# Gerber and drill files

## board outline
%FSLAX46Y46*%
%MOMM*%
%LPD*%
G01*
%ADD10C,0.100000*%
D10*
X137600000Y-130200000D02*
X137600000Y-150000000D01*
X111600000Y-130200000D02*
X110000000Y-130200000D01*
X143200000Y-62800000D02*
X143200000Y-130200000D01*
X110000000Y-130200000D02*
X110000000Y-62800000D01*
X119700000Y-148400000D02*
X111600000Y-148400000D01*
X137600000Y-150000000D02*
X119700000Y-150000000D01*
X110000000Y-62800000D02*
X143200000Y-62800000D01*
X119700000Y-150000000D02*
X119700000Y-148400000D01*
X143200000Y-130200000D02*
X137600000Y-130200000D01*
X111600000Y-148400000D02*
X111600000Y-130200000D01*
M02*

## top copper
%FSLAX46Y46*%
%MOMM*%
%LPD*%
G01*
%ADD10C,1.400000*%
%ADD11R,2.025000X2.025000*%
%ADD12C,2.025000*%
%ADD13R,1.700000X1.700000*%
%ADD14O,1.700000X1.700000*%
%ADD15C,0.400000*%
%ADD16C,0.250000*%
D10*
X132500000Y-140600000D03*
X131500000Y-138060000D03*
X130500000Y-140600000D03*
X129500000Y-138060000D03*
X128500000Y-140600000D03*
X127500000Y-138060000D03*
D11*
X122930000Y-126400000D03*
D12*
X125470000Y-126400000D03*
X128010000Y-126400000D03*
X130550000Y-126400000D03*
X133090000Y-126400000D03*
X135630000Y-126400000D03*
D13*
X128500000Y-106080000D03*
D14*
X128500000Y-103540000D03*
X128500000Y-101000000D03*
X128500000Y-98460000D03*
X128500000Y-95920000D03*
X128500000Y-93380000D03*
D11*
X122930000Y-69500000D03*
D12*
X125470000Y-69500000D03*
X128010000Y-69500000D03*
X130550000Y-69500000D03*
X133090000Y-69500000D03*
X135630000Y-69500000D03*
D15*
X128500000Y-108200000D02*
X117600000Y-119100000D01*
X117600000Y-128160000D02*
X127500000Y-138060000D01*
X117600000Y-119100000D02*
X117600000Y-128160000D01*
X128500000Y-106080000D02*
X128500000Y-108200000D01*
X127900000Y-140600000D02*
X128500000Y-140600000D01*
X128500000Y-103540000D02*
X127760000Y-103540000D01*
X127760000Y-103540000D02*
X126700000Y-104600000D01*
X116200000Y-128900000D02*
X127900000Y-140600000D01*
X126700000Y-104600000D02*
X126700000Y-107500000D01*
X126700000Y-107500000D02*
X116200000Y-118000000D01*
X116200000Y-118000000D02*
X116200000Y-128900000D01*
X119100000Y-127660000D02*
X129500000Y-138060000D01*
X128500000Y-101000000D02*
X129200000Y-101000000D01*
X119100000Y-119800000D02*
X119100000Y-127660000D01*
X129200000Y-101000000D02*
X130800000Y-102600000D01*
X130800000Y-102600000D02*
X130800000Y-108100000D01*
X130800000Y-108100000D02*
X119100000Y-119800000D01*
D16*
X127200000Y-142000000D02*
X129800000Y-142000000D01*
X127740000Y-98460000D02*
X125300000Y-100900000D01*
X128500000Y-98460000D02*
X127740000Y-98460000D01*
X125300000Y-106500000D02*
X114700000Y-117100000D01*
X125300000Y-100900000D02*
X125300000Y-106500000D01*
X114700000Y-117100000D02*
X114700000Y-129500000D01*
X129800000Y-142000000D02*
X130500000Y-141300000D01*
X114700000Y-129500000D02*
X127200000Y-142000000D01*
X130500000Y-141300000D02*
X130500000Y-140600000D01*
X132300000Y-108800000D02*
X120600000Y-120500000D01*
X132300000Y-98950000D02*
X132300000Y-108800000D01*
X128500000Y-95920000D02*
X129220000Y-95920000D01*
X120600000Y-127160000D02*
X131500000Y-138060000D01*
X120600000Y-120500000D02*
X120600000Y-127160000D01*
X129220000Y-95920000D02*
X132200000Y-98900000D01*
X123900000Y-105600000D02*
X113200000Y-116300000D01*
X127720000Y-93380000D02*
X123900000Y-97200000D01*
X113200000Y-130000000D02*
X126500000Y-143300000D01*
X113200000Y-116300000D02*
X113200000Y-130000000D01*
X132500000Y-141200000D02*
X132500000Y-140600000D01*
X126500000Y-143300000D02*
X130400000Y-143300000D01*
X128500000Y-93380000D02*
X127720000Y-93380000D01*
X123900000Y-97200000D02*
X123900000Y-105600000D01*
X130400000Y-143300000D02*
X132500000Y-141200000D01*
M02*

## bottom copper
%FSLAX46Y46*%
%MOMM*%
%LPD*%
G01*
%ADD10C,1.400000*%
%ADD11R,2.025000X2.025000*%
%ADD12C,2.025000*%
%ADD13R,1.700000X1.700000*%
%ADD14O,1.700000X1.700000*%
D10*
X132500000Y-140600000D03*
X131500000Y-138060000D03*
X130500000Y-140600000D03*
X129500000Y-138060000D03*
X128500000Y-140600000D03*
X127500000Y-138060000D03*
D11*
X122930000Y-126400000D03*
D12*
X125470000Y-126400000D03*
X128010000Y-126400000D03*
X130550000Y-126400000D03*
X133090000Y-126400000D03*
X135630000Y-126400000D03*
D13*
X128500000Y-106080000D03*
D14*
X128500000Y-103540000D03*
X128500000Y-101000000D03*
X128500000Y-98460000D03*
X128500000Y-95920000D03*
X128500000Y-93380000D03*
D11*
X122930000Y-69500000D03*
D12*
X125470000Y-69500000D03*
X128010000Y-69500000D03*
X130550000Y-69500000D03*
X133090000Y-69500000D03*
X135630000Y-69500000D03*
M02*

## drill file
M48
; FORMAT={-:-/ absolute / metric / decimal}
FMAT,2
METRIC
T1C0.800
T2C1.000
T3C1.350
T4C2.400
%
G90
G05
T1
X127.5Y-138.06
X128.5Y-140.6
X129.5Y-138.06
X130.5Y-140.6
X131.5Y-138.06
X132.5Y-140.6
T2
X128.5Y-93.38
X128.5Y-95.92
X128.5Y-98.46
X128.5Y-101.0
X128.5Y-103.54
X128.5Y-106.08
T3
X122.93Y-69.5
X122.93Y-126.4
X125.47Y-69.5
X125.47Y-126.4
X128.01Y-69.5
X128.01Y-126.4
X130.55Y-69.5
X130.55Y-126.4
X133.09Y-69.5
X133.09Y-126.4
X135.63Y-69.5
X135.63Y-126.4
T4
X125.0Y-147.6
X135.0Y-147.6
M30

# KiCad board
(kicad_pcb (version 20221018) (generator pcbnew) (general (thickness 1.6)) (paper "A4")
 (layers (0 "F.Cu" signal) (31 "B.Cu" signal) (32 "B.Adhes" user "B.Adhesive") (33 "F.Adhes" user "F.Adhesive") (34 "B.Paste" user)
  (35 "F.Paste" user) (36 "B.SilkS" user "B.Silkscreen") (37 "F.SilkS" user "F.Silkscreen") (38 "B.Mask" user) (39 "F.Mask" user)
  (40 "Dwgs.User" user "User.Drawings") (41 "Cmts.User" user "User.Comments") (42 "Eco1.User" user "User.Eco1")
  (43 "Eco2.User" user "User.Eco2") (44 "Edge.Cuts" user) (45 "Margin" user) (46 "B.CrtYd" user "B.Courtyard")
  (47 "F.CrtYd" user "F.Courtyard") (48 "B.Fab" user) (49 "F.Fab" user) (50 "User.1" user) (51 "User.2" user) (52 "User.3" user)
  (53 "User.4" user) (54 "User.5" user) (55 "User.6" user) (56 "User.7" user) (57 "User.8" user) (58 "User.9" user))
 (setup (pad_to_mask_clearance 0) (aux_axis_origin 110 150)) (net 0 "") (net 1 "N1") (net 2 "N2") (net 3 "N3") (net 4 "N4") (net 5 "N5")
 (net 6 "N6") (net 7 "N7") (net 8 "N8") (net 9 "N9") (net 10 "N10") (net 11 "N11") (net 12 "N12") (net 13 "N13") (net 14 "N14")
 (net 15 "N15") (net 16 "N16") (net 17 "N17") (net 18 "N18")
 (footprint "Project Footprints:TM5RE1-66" (layer "B.Cu") (at 130 147.6 180)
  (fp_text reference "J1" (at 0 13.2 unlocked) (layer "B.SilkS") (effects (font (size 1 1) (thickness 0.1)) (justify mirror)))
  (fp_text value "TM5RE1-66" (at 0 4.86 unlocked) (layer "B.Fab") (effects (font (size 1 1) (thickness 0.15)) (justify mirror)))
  (pad "" np_thru_hole circle (at -5 0 180) (size 2.4 2.4) (drill 2.4) (layers "F&B.Cu" "*.Mask"))
  (pad "" np_thru_hole circle (at 5 0 180) (size 2.4 2.4) (drill 2.4) (layers "F&B.Cu" "*.Mask"))
  (pad "1" thru_hole circle (at -2.5 7 180) (size 1.4 1.4) (drill 0.8) (layers "*.Cu" "*.Mask") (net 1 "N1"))
  (pad "2" thru_hole circle (at -1.5 9.54 180) (size 1.4 1.4) (drill 0.8) (layers "*.Cu" "*.Mask") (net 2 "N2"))
  (pad "3" thru_hole circle (at -0.5 7 180) (size 1.4 1.4) (drill 0.8) (layers "*.Cu" "*.Mask") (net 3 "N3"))
  (pad "4" thru_hole circle (at 0.5 9.54 180) (size 1.4 1.4) (drill 0.8) (layers "*.Cu" "*.Mask") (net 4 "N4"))
  (pad "5" thru_hole circle (at 1.5 7 180) (size 1.4 1.4) (drill 0.8) (layers "*.Cu" "*.Mask") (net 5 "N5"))
  (pad "6" thru_hole circle (at 2.5 9.54 180) (size 1.4 1.4) (drill 0.8) (layers "*.Cu" "*.Mask") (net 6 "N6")))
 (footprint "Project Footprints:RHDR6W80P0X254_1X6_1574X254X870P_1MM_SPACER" (layer "B.Cu") (at 122.93 126.4)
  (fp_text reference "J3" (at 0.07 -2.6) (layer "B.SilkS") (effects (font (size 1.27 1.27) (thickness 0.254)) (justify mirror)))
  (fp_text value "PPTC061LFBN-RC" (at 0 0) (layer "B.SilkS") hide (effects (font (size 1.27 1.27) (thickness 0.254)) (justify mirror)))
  (pad "1" thru_hole rect (at 0 0) (size 2.025 2.025) (drill 1.35) (layers "*.Cu" "*.Mask") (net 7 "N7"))
  (pad "2" thru_hole circle (at 2.54 0) (size 2.025 2.025) (drill 1.35) (layers "*.Cu" "*.Mask") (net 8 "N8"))
  (pad "3" thru_hole circle (at 5.08 0) (size 2.025 2.025) (drill 1.35) (layers "*.Cu" "*.Mask") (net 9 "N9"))
  (pad "4" thru_hole circle (at 7.62 0) (size 2.025 2.025) (drill 1.35) (layers "*.Cu" "*.Mask") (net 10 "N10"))
  (pad "5" thru_hole circle (at 10.16 0) (size 2.025 2.025) (drill 1.35) (layers "*.Cu" "*.Mask") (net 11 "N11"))
  (pad "6" thru_hole circle (at 12.7 0) (size 2.025 2.025) (drill 1.35) (layers "*.Cu" "*.Mask") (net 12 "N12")))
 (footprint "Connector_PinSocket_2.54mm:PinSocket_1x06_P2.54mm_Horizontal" (layer "B.Cu") (at 128.5 106.08)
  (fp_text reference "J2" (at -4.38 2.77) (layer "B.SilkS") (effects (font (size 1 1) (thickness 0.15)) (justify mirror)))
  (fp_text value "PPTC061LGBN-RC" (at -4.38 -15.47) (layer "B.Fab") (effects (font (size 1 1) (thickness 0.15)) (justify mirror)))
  (pad "1" thru_hole rect (at 0 0) (size 1.7 1.7) (drill 1) (layers "*.Cu" "*.Mask") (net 6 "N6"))
  (pad "2" thru_hole oval (at 0 -2.54) (size 1.7 1.7) (drill 1) (layers "*.Cu" "*.Mask") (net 5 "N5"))
  (pad "3" thru_hole oval (at 0 -5.08) (size 1.7 1.7) (drill 1) (layers "*.Cu" "*.Mask") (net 4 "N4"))
  (pad "4" thru_hole oval (at 0 -7.62) (size 1.7 1.7) (drill 1) (layers "*.Cu" "*.Mask") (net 3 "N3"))
  (pad "5" thru_hole oval (at 0 -10.16) (size 1.7 1.7) (drill 1) (layers "*.Cu" "*.Mask") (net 2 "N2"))
  (pad "6" thru_hole oval (at 0 -12.7) (size 1.7 1.7) (drill 1) (layers "*.Cu" "*.Mask") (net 1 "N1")))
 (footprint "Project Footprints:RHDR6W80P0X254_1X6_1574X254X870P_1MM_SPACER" (layer "B.Cu") (at 122.93 69.5)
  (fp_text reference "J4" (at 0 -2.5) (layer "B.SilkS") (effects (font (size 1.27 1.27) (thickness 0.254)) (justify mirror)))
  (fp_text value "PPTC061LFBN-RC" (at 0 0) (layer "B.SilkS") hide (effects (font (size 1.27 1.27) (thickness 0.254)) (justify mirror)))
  (pad "1" thru_hole rect (at 0 0) (size 2.025 2.025) (drill 1.35) (layers "*.Cu" "*.Mask") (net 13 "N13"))
  (pad "2" thru_hole circle (at 2.54 0) (size 2.025 2.025) (drill 1.35) (layers "*.Cu" "*.Mask") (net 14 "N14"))
  (pad "3" thru_hole circle (at 5.08 0) (size 2.025 2.025) (drill 1.35) (layers "*.Cu" "*.Mask") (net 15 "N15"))
  (pad "4" thru_hole circle (at 7.62 0) (size 2.025 2.025) (drill 1.35) (layers "*.Cu" "*.Mask") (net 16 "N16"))
  (pad "5" thru_hole circle (at 10.16 0) (size 2.025 2.025) (drill 1.35) (layers "*.Cu" "*.Mask") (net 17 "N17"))
  (pad "6" thru_hole circle (at 12.7 0) (size 2.025 2.025) (drill 1.35) (layers "*.Cu" "*.Mask") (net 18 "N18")))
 (gr_line (start 137.6 130.2) (end 137.6 150) (stroke (width 0.1) (type default)) (layer "Edge.Cuts"))
 (gr_line (start 111.6 130.2) (end 110 130.2) (stroke (width 0.1) (type default)) (layer "Edge.Cuts"))
 (gr_line (start 143.2 62.8) (end 143.2 130.2) (stroke (width 0.1) (type default)) (layer "Edge.Cuts"))
 (gr_line (start 110 130.2) (end 110 62.8) (stroke (width 0.1) (type default)) (layer "Edge.Cuts"))
 (gr_line (start 119.7 148.4) (end 111.6 148.4) (stroke (width 0.1) (type default)) (layer "Edge.Cuts"))
 (gr_line (start 137.6 150) (end 119.7 150) (stroke (width 0.1) (type default)) (layer "Edge.Cuts"))
 (gr_line (start 110 62.8) (end 143.2 62.8) (stroke (width 0.1) (type default)) (layer "Edge.Cuts"))
 (gr_line (start 119.7 150) (end 119.7 148.4) (stroke (width 0.1) (type default)) (layer "Edge.Cuts"))
 (gr_line (start 143.2 130.2) (end 137.6 130.2) (stroke (width 0.1) (type default)) (layer "Edge.Cuts"))
 (gr_line (start 111.6 148.4) (end 111.6 130.2) (stroke (width 0.1) (type default)) (layer "Edge.Cuts"))
 (segment (start 128.5 108.2) (end 117.6 119.1) (width 0.4) (layer "F.Cu") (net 6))
 (segment (start 117.6 128.16) (end 127.5 138.06) (width 0.4) (layer "F.Cu") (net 6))
 (segment (start 117.6 119.1) (end 117.6 128.16) (width 0.4) (layer "F.Cu") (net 6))
 (segment (start 128.5 106.08) (end 128.5 108.2) (width 0.4) (layer "F.Cu") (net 6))
 (segment (start 127.9 140.6) (end 128.5 140.6) (width 0.4) (layer "F.Cu") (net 5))
 (segment (start 128.5 103.54) (end 127.76 103.54) (width 0.4) (layer "F.Cu") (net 5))
 (segment (start 127.76 103.54) (end 126.7 104.6) (width 0.4) (layer "F.Cu") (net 5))
 (segment (start 116.2 128.9) (end 127.9 140.6) (width 0.4) (layer "F.Cu") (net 5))
 (segment (start 126.7 104.6) (end 126.7 107.5) (width 0.4) (layer "F.Cu") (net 5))
 (segment (start 126.7 107.5) (end 116.2 118) (width 0.4) (layer "F.Cu") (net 5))
 (segment (start 116.2 118) (end 116.2 128.9) (width 0.4) (layer "F.Cu") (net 5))
 (segment (start 119.1 127.66) (end 129.5 138.06) (width 0.4) (layer "F.Cu") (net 4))
 (segment (start 128.5 101) (end 129.2 101) (width 0.4) (layer "F.Cu") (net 4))
 (segment (start 119.1 119.8) (end 119.1 127.66) (width 0.4) (layer "F.Cu") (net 4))
 (segment (start 129.2 101) (end 130.8 102.6) (width 0.4) (layer "F.Cu") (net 4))
 (segment (start 130.8 102.6) (end 130.8 108.1) (width 0.4) (layer "F.Cu") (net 4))
 (segment (start 130.8 108.1) (end 119.1 119.8) (width 0.4) (layer "F.Cu") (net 4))
 (segment (start 127.2 142) (end 129.8 142) (width 0.25) (layer "F.Cu") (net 3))
 (segment (start 127.74 98.46) (end 125.3 100.9) (width 0.25) (layer "F.Cu") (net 3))
 (segment (start 128.5 98.46) (end 127.74 98.46) (width 0.25) (layer "F.Cu") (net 3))
 (segment (start 125.3 106.5) (end 114.7 117.1) (width 0.25) (layer "F.Cu") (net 3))
 (segment (start 125.3 100.9) (end 125.3 106.5) (width 0.25) (layer "F.Cu") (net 3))
 (segment (start 114.7 117.1) (end 114.7 129.5) (width 0.25) (layer "F.Cu") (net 3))
 (segment (start 129.8 142) (end 130.5 141.3) (width 0.25) (layer "F.Cu") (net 3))
 (segment (start 114.7 129.5) (end 127.2 142) (width 0.25) (layer "F.Cu") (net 3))
 (segment (start 130.5 141.3) (end 130.5 140.6) (width 0.25) (layer "F.Cu") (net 3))
 (segment (start 132.3 108.8) (end 120.6 120.5) (width 0.25) (layer "F.Cu") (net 2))
 (segment (start 132.3 98.95) (end 132.3 108.8) (width 0.25) (layer "F.Cu") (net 2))
 (segment (start 128.5 95.92) (end 129.22 95.92) (width 0.25) (layer "F.Cu") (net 2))
 (segment (start 120.6 127.16) (end 131.5 138.06) (width 0.25) (layer "F.Cu") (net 2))
 (segment (start 120.6 120.5) (end 120.6 127.16) (width 0.25) (layer "F.Cu") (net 2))
 (segment (start 129.22 95.92) (end 132.2 98.9) (width 0.25) (layer "F.Cu") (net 2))
 (segment (start 123.9 105.6) (end 113.2 116.3) (width 0.25) (layer "F.Cu") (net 1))
 (segment (start 127.72 93.38) (end 123.9 97.2) (width 0.25) (layer "F.Cu") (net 1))
 (segment (start 113.2 130) (end 126.5 143.3) (width 0.25) (layer "F.Cu") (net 1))
 (segment (start 113.2 116.3) (end 113.2 130) (width 0.25) (layer "F.Cu") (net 1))
 (segment (start 132.5 141.2) (end 132.5 140.6) (width 0.25) (layer "F.Cu") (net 1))
 (segment (start 126.5 143.3) (end 130.4 143.3) (width 0.25) (layer "F.Cu") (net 1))
 (segment (start 128.5 93.38) (end 127.72 93.38) (width 0.25) (layer "F.Cu") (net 1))
 (segment (start 123.9 97.2) (end 123.9 105.6) (width 0.25) (layer "F.Cu") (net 1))
 (segment (start 130.4 143.3) (end 132.5 141.2) (width 0.25) (layer "F.Cu") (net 1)))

